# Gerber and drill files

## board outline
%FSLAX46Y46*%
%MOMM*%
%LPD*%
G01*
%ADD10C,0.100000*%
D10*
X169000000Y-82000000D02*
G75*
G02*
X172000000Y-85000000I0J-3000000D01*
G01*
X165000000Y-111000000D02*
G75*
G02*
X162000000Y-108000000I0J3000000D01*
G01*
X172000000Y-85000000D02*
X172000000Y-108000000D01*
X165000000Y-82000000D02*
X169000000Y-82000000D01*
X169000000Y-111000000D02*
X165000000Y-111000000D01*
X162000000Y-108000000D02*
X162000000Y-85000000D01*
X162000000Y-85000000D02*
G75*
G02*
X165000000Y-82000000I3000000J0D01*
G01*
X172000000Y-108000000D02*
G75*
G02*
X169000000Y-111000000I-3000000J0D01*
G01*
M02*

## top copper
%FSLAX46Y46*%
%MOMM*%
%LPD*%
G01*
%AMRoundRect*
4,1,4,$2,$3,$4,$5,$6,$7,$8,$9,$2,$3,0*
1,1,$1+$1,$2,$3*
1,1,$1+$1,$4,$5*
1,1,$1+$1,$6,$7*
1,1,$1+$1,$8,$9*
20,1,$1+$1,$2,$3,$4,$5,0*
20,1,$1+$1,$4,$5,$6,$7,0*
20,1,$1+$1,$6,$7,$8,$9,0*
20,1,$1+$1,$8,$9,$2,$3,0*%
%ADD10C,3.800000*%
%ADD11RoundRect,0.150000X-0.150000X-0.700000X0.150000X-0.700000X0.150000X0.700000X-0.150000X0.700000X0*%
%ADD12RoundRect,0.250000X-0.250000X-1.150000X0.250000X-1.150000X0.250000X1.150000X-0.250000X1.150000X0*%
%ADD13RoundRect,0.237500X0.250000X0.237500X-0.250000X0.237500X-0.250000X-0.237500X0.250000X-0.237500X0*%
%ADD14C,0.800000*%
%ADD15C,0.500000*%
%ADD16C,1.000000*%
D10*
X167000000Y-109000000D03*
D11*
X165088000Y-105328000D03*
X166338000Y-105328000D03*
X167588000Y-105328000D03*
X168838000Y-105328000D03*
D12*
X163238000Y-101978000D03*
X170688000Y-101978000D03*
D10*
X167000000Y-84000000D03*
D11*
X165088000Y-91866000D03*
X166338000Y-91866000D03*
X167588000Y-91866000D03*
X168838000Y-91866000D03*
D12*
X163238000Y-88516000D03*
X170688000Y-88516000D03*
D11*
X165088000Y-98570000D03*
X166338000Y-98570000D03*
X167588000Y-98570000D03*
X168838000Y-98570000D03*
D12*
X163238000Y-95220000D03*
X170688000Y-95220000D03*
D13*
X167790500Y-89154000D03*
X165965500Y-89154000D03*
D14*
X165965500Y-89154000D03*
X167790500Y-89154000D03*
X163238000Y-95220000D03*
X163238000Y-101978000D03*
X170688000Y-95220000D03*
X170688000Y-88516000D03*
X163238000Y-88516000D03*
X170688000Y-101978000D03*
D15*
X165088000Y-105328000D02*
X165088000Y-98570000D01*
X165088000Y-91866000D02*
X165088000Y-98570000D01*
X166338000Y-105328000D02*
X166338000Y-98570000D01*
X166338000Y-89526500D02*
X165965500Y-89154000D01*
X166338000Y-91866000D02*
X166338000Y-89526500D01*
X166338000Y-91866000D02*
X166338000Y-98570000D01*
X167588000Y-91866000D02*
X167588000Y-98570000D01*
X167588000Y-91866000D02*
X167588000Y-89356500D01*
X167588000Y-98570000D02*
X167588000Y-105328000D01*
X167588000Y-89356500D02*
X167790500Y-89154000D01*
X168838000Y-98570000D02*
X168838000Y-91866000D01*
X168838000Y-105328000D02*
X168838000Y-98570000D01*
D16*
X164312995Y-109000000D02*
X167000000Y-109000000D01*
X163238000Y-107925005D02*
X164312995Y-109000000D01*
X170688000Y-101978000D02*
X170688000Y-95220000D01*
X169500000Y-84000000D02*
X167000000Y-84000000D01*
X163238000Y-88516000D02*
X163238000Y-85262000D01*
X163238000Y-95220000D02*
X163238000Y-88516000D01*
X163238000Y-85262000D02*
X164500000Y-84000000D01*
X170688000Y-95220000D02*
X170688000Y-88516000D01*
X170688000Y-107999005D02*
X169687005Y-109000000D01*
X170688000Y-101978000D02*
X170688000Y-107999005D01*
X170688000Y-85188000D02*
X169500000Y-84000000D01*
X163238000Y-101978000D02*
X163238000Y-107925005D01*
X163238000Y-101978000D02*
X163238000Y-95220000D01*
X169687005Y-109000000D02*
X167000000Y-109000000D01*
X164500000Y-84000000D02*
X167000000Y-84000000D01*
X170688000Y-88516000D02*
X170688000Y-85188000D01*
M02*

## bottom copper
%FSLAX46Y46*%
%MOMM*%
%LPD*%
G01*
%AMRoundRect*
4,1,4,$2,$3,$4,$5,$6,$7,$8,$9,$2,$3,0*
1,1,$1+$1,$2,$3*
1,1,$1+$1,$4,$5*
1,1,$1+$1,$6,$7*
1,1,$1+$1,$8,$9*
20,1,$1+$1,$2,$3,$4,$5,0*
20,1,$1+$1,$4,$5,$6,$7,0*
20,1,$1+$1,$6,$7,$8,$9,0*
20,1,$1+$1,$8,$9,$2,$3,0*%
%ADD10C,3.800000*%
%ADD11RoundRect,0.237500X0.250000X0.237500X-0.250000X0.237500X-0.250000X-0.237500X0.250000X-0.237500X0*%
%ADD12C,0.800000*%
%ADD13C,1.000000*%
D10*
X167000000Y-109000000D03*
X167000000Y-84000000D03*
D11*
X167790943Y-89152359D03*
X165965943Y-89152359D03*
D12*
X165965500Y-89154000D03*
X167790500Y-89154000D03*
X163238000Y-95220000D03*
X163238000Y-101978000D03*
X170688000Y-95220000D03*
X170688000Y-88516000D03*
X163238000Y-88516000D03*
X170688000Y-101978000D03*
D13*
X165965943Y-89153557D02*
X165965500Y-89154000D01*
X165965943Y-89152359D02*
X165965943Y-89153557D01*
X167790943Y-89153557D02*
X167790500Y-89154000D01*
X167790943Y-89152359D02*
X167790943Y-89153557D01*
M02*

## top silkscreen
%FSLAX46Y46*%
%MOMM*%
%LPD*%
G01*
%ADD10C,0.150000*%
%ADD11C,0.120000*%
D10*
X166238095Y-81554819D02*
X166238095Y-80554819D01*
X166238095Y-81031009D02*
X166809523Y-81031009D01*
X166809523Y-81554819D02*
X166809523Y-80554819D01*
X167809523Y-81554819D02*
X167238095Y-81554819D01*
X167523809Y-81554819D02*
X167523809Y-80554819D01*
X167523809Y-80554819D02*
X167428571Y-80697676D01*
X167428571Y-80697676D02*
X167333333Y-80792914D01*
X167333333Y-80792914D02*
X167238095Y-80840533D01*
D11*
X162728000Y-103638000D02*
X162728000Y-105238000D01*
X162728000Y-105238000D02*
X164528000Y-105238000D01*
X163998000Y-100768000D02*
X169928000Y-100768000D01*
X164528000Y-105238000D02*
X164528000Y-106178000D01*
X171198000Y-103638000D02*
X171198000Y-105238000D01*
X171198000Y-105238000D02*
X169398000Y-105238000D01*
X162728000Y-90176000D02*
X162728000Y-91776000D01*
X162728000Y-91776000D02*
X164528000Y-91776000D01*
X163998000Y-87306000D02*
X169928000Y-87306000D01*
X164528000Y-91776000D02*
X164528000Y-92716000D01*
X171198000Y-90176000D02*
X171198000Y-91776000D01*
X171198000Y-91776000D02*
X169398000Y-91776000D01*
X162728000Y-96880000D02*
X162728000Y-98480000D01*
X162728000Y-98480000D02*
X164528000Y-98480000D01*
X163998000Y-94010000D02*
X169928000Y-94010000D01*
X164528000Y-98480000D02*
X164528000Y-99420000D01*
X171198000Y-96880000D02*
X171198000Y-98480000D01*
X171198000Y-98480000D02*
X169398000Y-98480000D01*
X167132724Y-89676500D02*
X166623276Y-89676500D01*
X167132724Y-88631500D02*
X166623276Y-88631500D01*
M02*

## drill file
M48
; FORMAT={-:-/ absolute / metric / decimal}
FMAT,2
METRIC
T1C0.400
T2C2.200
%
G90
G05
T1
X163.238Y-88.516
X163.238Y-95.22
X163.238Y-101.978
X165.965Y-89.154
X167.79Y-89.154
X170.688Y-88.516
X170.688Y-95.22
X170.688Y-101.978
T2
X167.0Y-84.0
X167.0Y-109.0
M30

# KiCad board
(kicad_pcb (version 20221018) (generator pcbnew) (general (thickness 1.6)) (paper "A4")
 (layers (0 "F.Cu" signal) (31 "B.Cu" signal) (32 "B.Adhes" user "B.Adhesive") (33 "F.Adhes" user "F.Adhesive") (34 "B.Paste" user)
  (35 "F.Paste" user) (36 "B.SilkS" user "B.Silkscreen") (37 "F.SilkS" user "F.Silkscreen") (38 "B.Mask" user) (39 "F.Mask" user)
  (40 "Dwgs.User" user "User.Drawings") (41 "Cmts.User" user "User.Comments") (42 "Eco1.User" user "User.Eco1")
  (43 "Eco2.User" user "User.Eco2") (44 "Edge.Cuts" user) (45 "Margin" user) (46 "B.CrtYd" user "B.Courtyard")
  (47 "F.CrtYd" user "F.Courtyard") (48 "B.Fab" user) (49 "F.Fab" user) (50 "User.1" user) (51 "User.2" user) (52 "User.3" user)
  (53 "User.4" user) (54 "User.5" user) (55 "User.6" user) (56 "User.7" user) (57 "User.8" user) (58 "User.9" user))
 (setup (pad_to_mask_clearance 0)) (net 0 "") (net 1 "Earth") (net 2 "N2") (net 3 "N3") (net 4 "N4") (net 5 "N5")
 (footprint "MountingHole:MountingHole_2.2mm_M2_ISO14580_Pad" (layer "F.Cu") (at 167 109)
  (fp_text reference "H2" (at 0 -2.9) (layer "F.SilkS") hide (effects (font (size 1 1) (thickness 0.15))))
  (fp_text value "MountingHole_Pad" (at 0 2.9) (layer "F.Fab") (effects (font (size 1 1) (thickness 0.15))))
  (pad "1" thru_hole circle (at 0 0) (size 3.8 3.8) (drill 2.2) (layers "*.Cu" "*.Mask") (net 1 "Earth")))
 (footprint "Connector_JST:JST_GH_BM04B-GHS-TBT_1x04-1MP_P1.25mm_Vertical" (layer "F.Cu") (at 166.963 103.378)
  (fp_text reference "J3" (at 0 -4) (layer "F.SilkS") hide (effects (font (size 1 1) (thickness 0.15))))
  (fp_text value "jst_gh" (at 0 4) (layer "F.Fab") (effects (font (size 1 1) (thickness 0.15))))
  (fp_line (start -4.235 0.26) (end -4.235 1.86) (stroke (width 0.12) (type solid)) (layer "F.SilkS"))
  (fp_line (start -4.235 1.86) (end -2.435 1.86) (stroke (width 0.12) (type solid)) (layer "F.SilkS"))
  (fp_line (start -2.965 -2.61) (end 2.965 -2.61) (stroke (width 0.12) (type solid)) (layer "F.SilkS"))
  (fp_line (start -2.435 1.86) (end -2.435 2.8) (stroke (width 0.12) (type solid)) (layer "F.SilkS"))
  (fp_line (start 4.235 0.26) (end 4.235 1.86) (stroke (width 0.12) (type solid)) (layer "F.SilkS"))
  (fp_line (start 4.235 1.86) (end 2.435 1.86) (stroke (width 0.12) (type solid)) (layer "F.SilkS"))
  (pad "1" smd roundrect (at -1.875 1.95) (size 0.6 1.7) (layers "F.Cu" "F.Paste" "F.Mask") (roundrect_rratio 0.25) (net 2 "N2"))
  (pad "2" smd roundrect (at -0.625 1.95) (size 0.6 1.7) (layers "F.Cu" "F.Paste" "F.Mask") (roundrect_rratio 0.25) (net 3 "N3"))
  (pad "3" smd roundrect (at 0.625 1.95) (size 0.6 1.7) (layers "F.Cu" "F.Paste" "F.Mask") (roundrect_rratio 0.25) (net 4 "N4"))
  (pad "4" smd roundrect (at 1.875 1.95) (size 0.6 1.7) (layers "F.Cu" "F.Paste" "F.Mask") (roundrect_rratio 0.25) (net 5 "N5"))
  (pad "MP" smd roundrect (at -3.725 -1.4) (size 1 2.8) (layers "F.Cu" "F.Paste" "F.Mask") (roundrect_rratio 0.25) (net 1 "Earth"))
  (pad "MP" smd roundrect (at 3.725 -1.4) (size 1 2.8) (layers "F.Cu" "F.Paste" "F.Mask") (roundrect_rratio 0.25) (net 1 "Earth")))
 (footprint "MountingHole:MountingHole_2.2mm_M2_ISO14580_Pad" (layer "F.Cu") (at 167 84)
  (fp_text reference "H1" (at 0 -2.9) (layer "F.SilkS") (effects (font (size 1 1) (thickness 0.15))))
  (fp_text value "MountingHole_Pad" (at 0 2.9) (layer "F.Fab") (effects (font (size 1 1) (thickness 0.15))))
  (pad "1" thru_hole circle (at 0 0) (size 3.8 3.8) (drill 2.2) (layers "*.Cu" "*.Mask") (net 1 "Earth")))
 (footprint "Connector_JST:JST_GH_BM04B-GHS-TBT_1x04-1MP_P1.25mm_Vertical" (layer "F.Cu") (at 166.963 89.916)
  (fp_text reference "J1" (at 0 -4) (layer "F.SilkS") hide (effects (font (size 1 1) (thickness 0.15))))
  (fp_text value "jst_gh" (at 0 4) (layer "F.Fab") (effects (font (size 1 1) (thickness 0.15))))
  (fp_line (start -4.235 0.26) (end -4.235 1.86) (stroke (width 0.12) (type solid)) (layer "F.SilkS"))
  (fp_line (start -4.235 1.86) (end -2.435 1.86) (stroke (width 0.12) (type solid)) (layer "F.SilkS"))
  (fp_line (start -2.965 -2.61) (end 2.965 -2.61) (stroke (width 0.12) (type solid)) (layer "F.SilkS"))
  (fp_line (start -2.435 1.86) (end -2.435 2.8) (stroke (width 0.12) (type solid)) (layer "F.SilkS"))
  (fp_line (start 4.235 0.26) (end 4.235 1.86) (stroke (width 0.12) (type solid)) (layer "F.SilkS"))
  (fp_line (start 4.235 1.86) (end 2.435 1.86) (stroke (width 0.12) (type solid)) (layer "F.SilkS"))
  (pad "1" smd roundrect (at -1.875 1.95) (size 0.6 1.7) (layers "F.Cu" "F.Paste" "F.Mask") (roundrect_rratio 0.25) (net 2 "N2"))
  (pad "2" smd roundrect (at -0.625 1.95) (size 0.6 1.7) (layers "F.Cu" "F.Paste" "F.Mask") (roundrect_rratio 0.25) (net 3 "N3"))
  (pad "3" smd roundrect (at 0.625 1.95) (size 0.6 1.7) (layers "F.Cu" "F.Paste" "F.Mask") (roundrect_rratio 0.25) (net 4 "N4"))
  (pad "4" smd roundrect (at 1.875 1.95) (size 0.6 1.7) (layers "F.Cu" "F.Paste" "F.Mask") (roundrect_rratio 0.25) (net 5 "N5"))
  (pad "MP" smd roundrect (at -3.725 -1.4) (size 1 2.8) (layers "F.Cu" "F.Paste" "F.Mask") (roundrect_rratio 0.25) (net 1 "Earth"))
  (pad "MP" smd roundrect (at 3.725 -1.4) (size 1 2.8) (layers "F.Cu" "F.Paste" "F.Mask") (roundrect_rratio 0.25) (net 1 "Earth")))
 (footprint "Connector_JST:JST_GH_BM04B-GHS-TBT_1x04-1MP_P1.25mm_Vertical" (layer "F.Cu") (at 166.963 96.62)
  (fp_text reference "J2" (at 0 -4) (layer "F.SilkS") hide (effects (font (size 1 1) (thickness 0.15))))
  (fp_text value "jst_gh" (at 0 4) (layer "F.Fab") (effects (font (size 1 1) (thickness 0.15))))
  (fp_line (start -4.235 0.26) (end -4.235 1.86) (stroke (width 0.12) (type solid)) (layer "F.SilkS"))
  (fp_line (start -4.235 1.86) (end -2.435 1.86) (stroke (width 0.12) (type solid)) (layer "F.SilkS"))
  (fp_line (start -2.965 -2.61) (end 2.965 -2.61) (stroke (width 0.12) (type solid)) (layer "F.SilkS"))
  (fp_line (start -2.435 1.86) (end -2.435 2.8) (stroke (width 0.12) (type solid)) (layer "F.SilkS"))
  (fp_line (start 4.235 0.26) (end 4.235 1.86) (stroke (width 0.12) (type solid)) (layer "F.SilkS"))
  (fp_line (start 4.235 1.86) (end 2.435 1.86) (stroke (width 0.12) (type solid)) (layer "F.SilkS"))
  (pad "1" smd roundrect (at -1.875 1.95) (size 0.6 1.7) (layers "F.Cu" "F.Paste" "F.Mask") (roundrect_rratio 0.25) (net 2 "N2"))
  (pad "2" smd roundrect (at -0.625 1.95) (size 0.6 1.7) (layers "F.Cu" "F.Paste" "F.Mask") (roundrect_rratio 0.25) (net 3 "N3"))
  (pad "3" smd roundrect (at 0.625 1.95) (size 0.6 1.7) (layers "F.Cu" "F.Paste" "F.Mask") (roundrect_rratio 0.25) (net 4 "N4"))
  (pad "4" smd roundrect (at 1.875 1.95) (size 0.6 1.7) (layers "F.Cu" "F.Paste" "F.Mask") (roundrect_rratio 0.25) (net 5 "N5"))
  (pad "MP" smd roundrect (at -3.725 -1.4) (size 1 2.8) (layers "F.Cu" "F.Paste" "F.Mask") (roundrect_rratio 0.25) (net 1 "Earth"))
  (pad "MP" smd roundrect (at 3.725 -1.4) (size 1 2.8) (layers "F.Cu" "F.Paste" "F.Mask") (roundrect_rratio 0.25) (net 1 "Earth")))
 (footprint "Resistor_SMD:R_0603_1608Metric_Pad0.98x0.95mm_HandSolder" (layer "F.Cu") (at 166.878 89.154 180)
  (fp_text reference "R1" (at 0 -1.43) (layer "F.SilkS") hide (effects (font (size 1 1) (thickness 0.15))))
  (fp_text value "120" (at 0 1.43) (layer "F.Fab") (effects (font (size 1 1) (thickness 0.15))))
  (fp_line (start -0.254724 -0.5225) (end 0.254724 -0.5225) (stroke (width 0.12) (type solid)) (layer "F.SilkS"))
  (fp_line (start -0.254724 0.5225) (end 0.254724 0.5225) (stroke (width 0.12) (type solid)) (layer "F.SilkS"))
  (pad "1" smd roundrect (at -0.9125 0 180) (size 0.975 0.95) (layers "F.Cu" "F.Paste" "F.Mask") (roundrect_rratio 0.25) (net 4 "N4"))
  (pad "2" smd roundrect (at 0.9125 0 180) (size 0.975 0.95) (layers "F.Cu" "F.Paste" "F.Mask") (roundrect_rratio 0.25) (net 3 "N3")))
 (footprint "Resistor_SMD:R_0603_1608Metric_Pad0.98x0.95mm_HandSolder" (layer "B.Cu") (at 166.878443 89.152359 180)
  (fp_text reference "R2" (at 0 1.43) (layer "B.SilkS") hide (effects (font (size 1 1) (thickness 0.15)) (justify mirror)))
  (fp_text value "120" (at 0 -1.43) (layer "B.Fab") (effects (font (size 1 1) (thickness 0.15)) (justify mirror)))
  (pad "1" smd roundrect (at -0.9125 0 180) (size 0.975 0.95) (layers "B.Cu" "B.Paste" "B.Mask") (roundrect_rratio 0.25) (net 4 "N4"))
  (pad "2" smd roundrect (at 0.9125 0 180) (size 0.975 0.95) (layers "B.Cu" "B.Paste" "B.Mask") (roundrect_rratio 0.25) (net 3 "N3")))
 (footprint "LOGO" (layer "B.Cu") (at 166.963 96 -90)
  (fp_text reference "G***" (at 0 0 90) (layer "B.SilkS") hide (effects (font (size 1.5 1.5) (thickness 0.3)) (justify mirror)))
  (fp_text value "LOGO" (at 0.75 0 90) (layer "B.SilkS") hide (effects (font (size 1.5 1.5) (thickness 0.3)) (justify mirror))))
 (gr_arc (start 169 82) (mid 171.12132 82.87868) (end 172 85) (stroke (width 0.1) (type default)) (layer "Edge.Cuts"))
 (gr_arc (start 165 111) (mid 162.87868 110.12132) (end 162 108) (stroke (width 0.1) (type default)) (layer "Edge.Cuts"))
 (gr_line (start 172 85) (end 172 108) (stroke (width 0.1) (type default)) (layer "Edge.Cuts"))
 (gr_line (start 165 82) (end 169 82) (stroke (width 0.1) (type default)) (layer "Edge.Cuts"))
 (gr_line (start 169 111) (end 165 111) (stroke (width 0.1) (type default)) (layer "Edge.Cuts"))
 (gr_line (start 162 108) (end 162 85) (stroke (width 0.1) (type default)) (layer "Edge.Cuts"))
 (gr_arc (start 162 85) (mid 162.87868 82.87868) (end 165 82) (stroke (width 0.1) (type default)) (layer "Edge.Cuts"))
 (gr_arc (start 172 108) (mid 171.12132 110.12132) (end 169 111) (stroke (width 0.1) (type default)) (layer "Edge.Cuts"))
 (segment (start 165.088 105.328) (end 165.088 98.57) (width 0.5) (layer "F.Cu") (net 2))
 (segment (start 165.088 91.866) (end 165.088 98.57) (width 0.5) (layer "F.Cu") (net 2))
 (segment (start 166.338 105.328) (end 166.338 98.57) (width 0.5) (layer "F.Cu") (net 3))
 (segment (start 166.338 89.5265) (end 165.9655 89.154) (width 0.5) (layer "F.Cu") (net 3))
 (segment (start 166.338 91.866) (end 166.338 89.5265) (width 0.5) (layer "F.Cu") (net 3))
 (segment (start 166.338 91.866) (end 166.338 98.57) (width 0.5) (layer "F.Cu") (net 3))
 (via (at 165.9655 89.154) (size 0.8) (drill 0.4) (layers "F.Cu" "B.Cu") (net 3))
 (segment (start 165.965943 89.153557) (end 165.9655 89.154) (width 1) (layer "B.Cu") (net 3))
 (segment (start 165.965943 89.152359) (end 165.965943 89.153557) (width 1) (layer "B.Cu") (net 3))
 (segment (start 167.588 91.866) (end 167.588 98.57) (width 0.5) (layer "F.Cu") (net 4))
 (segment (start 167.588 91.866) (end 167.588 89.3565) (width 0.5) (layer "F.Cu") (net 4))
 (segment (start 167.588 98.57) (end 167.588 105.328) (width 0.5) (layer "F.Cu") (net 4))
 (segment (start 167.588 89.3565) (end 167.7905 89.154) (width 0.5) (layer "F.Cu") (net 4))
 (via (at 167.7905 89.154) (size 0.8) (drill 0.4) (layers "F.Cu" "B.Cu") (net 4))
 (segment (start 167.790943 89.153557) (end 167.7905 89.154) (width 1) (layer "B.Cu") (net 4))
 (segment (start 167.790943 89.152359) (end 167.790943 89.153557) (width 1) (layer "B.Cu") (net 4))
 (segment (start 168.838 98.57) (end 168.838 91.866) (width 0.5) (layer "F.Cu") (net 5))
 (segment (start 168.838 105.328) (end 168.838 98.57) (width 0.5) (layer "F.Cu") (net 5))
 (segment (start 164.312995 109) (end 167 109) (width 1) (layer "F.Cu") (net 1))
 (segment (start 163.238 107.925005) (end 164.312995 109) (width 1) (layer "F.Cu") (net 1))
 (segment (start 170.688 101.978) (end 170.688 95.22) (width 1) (layer "F.Cu") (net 1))
 (segment (start 169.5 84) (end 167 84) (width 1) (layer "F.Cu") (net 1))
 (segment (start 163.238 88.516) (end 163.238 85.262) (width 1) (layer "F.Cu") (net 1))
 (segment (start 163.238 95.22) (end 163.238 88.516) (width 1) (layer "F.Cu") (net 1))
 (segment (start 163.238 85.262) (end 164.5 84) (width 1) (layer "F.Cu") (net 1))
 (segment (start 170.688 95.22) (end 170.688 88.516) (width 1) (layer "F.Cu") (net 1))
 (segment (start 170.688 107.999005) (end 169.687005 109) (width 1) (layer "F.Cu") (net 1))
 (segment (start 170.688 101.978) (end 170.688 107.999005) (width 1) (layer "F.Cu") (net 1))
 (segment (start 170.688 85.188) (end 169.5 84) (width 1) (layer "F.Cu") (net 1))
 (segment (start 163.238 101.978) (end 163.238 107.925005) (width 1) (layer "F.Cu") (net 1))
 (segment (start 163.238 101.978) (end 163.238 95.22) (width 1) (layer "F.Cu") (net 1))
 (segment (start 169.687005 109) (end 167 109) (width 1) (layer "F.Cu") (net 1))
 (segment (start 164.5 84) (end 167 84) (width 1) (layer "F.Cu") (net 1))
 (segment (start 170.688 88.516) (end 170.688 85.188) (width 1) (layer "F.Cu") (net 1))
 (via (at 163.238 95.22) (size 0.8) (drill 0.4) (layers "F.Cu" "B.Cu") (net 1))
 (via (at 163.238 101.978) (size 0.8) (drill 0.4) (layers "F.Cu" "B.Cu") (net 1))
 (via (at 170.688 95.22) (size 0.8) (drill 0.4) (layers "F.Cu" "B.Cu") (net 1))
 (via (at 170.688 88.516) (size 0.8) (drill 0.4) (layers "F.Cu" "B.Cu") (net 1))
 (via (at 163.238 88.516) (size 0.8) (drill 0.4) (layers "F.Cu" "B.Cu") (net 1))
 (via (at 170.688 101.978) (size 0.8) (drill 0.4) (layers "F.Cu" "B.Cu") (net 1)))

